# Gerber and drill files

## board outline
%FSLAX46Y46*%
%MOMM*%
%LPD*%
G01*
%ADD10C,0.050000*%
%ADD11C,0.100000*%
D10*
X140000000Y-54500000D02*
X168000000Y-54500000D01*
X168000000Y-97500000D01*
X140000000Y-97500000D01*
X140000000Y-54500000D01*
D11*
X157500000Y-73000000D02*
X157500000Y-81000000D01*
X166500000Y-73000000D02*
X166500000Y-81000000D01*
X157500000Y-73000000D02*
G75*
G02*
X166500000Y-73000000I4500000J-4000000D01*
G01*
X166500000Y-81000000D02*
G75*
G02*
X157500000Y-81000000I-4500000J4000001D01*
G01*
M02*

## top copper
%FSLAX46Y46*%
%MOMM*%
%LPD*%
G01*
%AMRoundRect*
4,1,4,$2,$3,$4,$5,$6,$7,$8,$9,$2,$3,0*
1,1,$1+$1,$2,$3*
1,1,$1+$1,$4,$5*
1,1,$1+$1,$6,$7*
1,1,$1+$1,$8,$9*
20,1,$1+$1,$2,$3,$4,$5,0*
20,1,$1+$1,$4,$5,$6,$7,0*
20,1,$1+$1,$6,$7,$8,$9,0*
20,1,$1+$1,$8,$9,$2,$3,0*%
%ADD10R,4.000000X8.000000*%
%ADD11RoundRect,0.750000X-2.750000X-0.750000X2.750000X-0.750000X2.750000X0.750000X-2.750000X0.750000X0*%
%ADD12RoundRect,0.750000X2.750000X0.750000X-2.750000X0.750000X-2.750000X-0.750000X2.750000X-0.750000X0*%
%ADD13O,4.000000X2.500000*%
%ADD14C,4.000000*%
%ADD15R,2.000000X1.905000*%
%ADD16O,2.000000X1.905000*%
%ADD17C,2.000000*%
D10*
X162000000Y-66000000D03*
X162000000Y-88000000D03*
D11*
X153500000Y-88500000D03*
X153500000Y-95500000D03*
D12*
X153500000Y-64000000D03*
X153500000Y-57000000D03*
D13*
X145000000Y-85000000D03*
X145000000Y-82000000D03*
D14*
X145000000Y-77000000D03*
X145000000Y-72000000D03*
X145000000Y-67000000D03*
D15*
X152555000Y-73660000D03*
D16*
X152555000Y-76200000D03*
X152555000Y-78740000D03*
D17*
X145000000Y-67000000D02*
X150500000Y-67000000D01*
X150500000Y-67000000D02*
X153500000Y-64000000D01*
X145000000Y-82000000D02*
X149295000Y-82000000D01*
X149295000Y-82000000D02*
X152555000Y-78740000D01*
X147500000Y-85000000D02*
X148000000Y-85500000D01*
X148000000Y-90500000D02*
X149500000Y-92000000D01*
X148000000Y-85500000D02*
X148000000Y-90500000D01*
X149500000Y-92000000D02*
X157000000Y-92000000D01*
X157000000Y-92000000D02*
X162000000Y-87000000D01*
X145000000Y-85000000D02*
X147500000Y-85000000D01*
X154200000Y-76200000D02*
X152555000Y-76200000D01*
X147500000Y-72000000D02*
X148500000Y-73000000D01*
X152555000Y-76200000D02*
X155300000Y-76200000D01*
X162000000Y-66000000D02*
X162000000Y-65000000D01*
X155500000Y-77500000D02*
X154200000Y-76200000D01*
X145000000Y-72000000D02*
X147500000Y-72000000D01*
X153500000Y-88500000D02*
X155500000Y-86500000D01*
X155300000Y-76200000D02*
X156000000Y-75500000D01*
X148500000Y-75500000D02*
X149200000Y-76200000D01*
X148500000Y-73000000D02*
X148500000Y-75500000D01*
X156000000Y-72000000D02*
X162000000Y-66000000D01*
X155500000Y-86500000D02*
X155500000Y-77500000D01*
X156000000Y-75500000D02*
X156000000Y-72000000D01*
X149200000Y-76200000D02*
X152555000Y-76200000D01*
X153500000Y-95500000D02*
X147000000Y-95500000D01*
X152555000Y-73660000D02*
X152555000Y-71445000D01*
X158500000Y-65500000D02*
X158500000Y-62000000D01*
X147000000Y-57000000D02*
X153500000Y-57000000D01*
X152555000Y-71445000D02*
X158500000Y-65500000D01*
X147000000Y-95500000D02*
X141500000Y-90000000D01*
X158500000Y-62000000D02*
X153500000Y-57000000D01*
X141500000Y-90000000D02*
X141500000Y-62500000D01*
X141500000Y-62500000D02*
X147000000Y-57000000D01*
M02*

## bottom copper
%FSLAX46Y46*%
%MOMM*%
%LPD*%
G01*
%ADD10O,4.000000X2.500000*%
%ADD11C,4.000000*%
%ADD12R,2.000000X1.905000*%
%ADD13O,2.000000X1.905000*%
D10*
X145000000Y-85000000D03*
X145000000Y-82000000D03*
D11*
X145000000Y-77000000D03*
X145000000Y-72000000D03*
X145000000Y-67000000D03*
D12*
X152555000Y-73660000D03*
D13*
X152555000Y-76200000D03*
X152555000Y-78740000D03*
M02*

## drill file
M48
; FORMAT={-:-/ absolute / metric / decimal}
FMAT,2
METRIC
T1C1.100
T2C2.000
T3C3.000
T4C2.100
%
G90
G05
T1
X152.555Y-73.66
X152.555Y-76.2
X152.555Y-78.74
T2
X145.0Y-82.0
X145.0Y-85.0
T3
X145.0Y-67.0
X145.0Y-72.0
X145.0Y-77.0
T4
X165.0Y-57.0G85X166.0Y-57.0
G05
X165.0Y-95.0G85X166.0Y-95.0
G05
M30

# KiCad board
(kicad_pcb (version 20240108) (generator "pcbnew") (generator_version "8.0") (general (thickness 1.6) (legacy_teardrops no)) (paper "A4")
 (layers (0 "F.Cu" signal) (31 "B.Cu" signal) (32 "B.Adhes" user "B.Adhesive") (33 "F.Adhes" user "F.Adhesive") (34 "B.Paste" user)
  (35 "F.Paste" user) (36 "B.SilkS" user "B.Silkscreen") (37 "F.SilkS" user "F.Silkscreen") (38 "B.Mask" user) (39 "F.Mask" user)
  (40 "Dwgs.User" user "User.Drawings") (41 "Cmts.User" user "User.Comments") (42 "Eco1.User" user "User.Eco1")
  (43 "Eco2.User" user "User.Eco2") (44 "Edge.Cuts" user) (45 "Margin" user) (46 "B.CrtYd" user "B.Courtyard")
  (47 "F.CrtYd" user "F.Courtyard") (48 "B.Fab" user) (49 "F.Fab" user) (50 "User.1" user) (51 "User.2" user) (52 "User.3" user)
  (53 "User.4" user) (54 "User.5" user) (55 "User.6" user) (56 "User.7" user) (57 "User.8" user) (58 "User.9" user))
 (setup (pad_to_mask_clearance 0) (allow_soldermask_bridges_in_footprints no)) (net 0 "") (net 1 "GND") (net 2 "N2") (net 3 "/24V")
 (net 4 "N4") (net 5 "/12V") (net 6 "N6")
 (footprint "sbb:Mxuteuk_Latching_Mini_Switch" (layer "F.Cu") (at 162 77 -90)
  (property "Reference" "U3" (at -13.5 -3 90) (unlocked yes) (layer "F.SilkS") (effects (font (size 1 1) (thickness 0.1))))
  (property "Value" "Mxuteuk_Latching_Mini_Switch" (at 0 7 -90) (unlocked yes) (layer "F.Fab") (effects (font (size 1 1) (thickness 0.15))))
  (fp_line (start -4 4.5) (end 4 4.5) (stroke (width 0.1) (type default)) (layer "Edge.Cuts"))
  (fp_line (start -4 -4.5) (end 4 -4.5) (stroke (width 0.1) (type default)) (layer "Edge.Cuts"))
  (fp_arc (start -4 4.5) (mid -6.020797 0) (end -4 -4.5) (stroke (width 0.1) (type default)) (layer "Edge.Cuts"))
  (fp_arc (start 4 -4.5) (mid 6.020797 0) (end 4 4.5) (stroke (width 0.1) (type default)) (layer "Edge.Cuts"))
  (pad "1" smd rect (at -11 0 270) (size 8 4) (layers "F.Cu" "F.Paste" "F.Mask") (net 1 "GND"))
  (pad "2" smd rect (at 11 0 270) (size 8 4) (layers "F.Cu" "F.Paste" "F.Mask") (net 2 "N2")))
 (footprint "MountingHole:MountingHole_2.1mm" (layer "F.Cu") (at 165.5 57)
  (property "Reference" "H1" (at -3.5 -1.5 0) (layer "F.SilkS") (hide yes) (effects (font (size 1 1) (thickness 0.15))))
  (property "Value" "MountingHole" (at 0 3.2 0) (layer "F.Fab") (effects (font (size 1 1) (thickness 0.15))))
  (pad "" np_thru_hole oval (at 0 0) (size 3.1 2.1) (drill oval 3.1 2.1) (layers "F&B.Cu" "*.Mask")))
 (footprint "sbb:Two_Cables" (layer "F.Cu") (at 153.5 92.5)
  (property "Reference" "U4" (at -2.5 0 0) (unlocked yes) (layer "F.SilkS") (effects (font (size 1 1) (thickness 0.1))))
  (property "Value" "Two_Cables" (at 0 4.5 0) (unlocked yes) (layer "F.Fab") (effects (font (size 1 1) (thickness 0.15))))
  (pad "1" smd roundrect (at 0 -4) (size 7 3) (layers "F.Cu" "F.Paste" "F.Mask") (roundrect_rratio 0.25) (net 1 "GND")
   (thermal_bridge_angle 45))
  (pad "2" smd roundrect (at 0 3) (size 7 3) (layers "F.Cu" "F.Paste" "F.Mask") (roundrect_rratio 0.25) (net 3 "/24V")
   (thermal_bridge_angle 45)))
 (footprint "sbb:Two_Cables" (layer "F.Cu") (at 153.5 60 180)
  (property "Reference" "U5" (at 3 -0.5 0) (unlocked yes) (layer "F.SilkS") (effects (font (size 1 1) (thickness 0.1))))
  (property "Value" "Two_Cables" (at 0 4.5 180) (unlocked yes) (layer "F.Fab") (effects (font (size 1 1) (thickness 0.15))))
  (pad "1" smd roundrect (at 0 -4 180) (size 7 3) (layers "F.Cu" "F.Paste" "F.Mask") (roundrect_rratio 0.25) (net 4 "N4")
   (thermal_bridge_angle 45))
  (pad "2" smd roundrect (at 0 3 180) (size 7 3) (layers "F.Cu" "F.Paste" "F.Mask") (roundrect_rratio 0.25) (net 3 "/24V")
   (thermal_bridge_angle 45)))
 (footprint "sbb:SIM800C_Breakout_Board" (layer "F.Cu") (at 145 85)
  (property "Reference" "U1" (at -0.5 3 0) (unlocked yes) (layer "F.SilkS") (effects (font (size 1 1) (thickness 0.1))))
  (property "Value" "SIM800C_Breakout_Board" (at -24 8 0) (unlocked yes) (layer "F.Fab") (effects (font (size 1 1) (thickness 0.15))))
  (pad "1" thru_hole oval (at 0 0) (size 4 2.5) (drill 2) (layers "*.Cu" "*.Mask") (remove_unused_layers no) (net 2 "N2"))
  (pad "2" thru_hole oval (at 0 -3) (size 4 2.5) (drill 2) (layers "*.Cu" "*.Mask") (remove_unused_layers no) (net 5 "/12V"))
  (pad "3" thru_hole circle (at 0 -8) (size 4 4) (drill 3) (layers "*.Cu" "*.Mask") (remove_unused_layers no) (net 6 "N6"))
  (pad "4" thru_hole circle (at 0 -13) (size 4 4) (drill 3) (layers "*.Cu" "*.Mask") (remove_unused_layers no) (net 1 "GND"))
  (pad "5" thru_hole circle (at 0 -18) (size 4 4) (drill 3) (layers "*.Cu" "*.Mask") (remove_unused_layers no) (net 4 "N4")))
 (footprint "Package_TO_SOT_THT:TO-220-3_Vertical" (layer "F.Cu") (at 152.555 73.66 -90)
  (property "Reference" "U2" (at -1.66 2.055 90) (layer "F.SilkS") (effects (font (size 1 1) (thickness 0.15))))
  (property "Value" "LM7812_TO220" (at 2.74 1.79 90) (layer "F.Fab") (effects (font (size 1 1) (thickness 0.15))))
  (pad "1" thru_hole rect (at 0 0 270) (size 1.905 2) (drill 1.1) (layers "*.Cu" "*.Mask") (remove_unused_layers no) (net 3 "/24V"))
  (pad "2" thru_hole oval (at 2.54 0 270) (size 1.905 2) (drill 1.1) (layers "*.Cu" "*.Mask") (remove_unused_layers no) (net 1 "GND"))
  (pad "3" thru_hole oval (at 5.08 0 270) (size 1.905 2) (drill 1.1) (layers "*.Cu" "*.Mask") (remove_unused_layers no) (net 5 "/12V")))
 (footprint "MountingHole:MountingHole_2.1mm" (layer "F.Cu") (at 165.5 95)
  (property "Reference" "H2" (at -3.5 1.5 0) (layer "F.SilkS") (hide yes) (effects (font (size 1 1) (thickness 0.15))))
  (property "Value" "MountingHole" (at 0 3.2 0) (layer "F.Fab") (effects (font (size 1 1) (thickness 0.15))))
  (pad "" np_thru_hole oval (at 0 0) (size 3.1 2.1) (drill oval 3.1 2.1) (layers "F&B.Cu" "*.Mask")))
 (gr_rect (start 140 54.5) (end 168 97.5) (stroke (width 0.05) (type default)) (fill none) (layer "Edge.Cuts"))
 (segment (start 145 67) (end 150.5 67) (width 2) (layer "F.Cu") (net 4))
 (segment (start 150.5 67) (end 153.5 64) (width 2) (layer "F.Cu") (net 4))
 (segment (start 145 82) (end 149.295 82) (width 2) (layer "F.Cu") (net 5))
 (segment (start 149.295 82) (end 152.555 78.74) (width 2) (layer "F.Cu") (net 5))
 (segment (start 147.5 85) (end 148 85.5) (width 2) (layer "F.Cu") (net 2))
 (segment (start 148 90.5) (end 149.5 92) (width 2) (layer "F.Cu") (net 2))
 (segment (start 148 85.5) (end 148 90.5) (width 2) (layer "F.Cu") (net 2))
 (segment (start 149.5 92) (end 157 92) (width 2) (layer "F.Cu") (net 2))
 (segment (start 157 92) (end 162 87) (width 2) (layer "F.Cu") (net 2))
 (segment (start 145 85) (end 147.5 85) (width 2) (layer "F.Cu") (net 2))
 (segment (start 154.2 76.2) (end 152.555 76.2) (width 2) (layer "F.Cu") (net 1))
 (segment (start 147.5 72) (end 148.5 73) (width 2) (layer "F.Cu") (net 1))
 (segment (start 152.555 76.2) (end 155.3 76.2) (width 2) (layer "F.Cu") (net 1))
 (segment (start 162 66) (end 162 65) (width 2) (layer "F.Cu") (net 1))
 (segment (start 155.5 77.5) (end 154.2 76.2) (width 2) (layer "F.Cu") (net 1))
 (segment (start 145 72) (end 147.5 72) (width 2) (layer "F.Cu") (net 1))
 (segment (start 153.5 88.5) (end 155.5 86.5) (width 2) (layer "F.Cu") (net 1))
 (segment (start 155.3 76.2) (end 156 75.5) (width 2) (layer "F.Cu") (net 1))
 (segment (start 148.5 75.5) (end 149.2 76.2) (width 2) (layer "F.Cu") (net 1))
 (segment (start 148.5 73) (end 148.5 75.5) (width 2) (layer "F.Cu") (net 1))
 (segment (start 156 72) (end 162 66) (width 2) (layer "F.Cu") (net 1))
 (segment (start 155.5 86.5) (end 155.5 77.5) (width 2) (layer "F.Cu") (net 1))
 (segment (start 156 75.5) (end 156 72) (width 2) (layer "F.Cu") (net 1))
 (segment (start 149.2 76.2) (end 152.555 76.2) (width 2) (layer "F.Cu") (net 1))
 (segment (start 153.5 95.5) (end 147 95.5) (width 2) (layer "F.Cu") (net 3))
 (segment (start 152.555 73.66) (end 152.555 71.445) (width 2) (layer "F.Cu") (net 3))
 (segment (start 158.5 65.5) (end 158.5 62) (width 2) (layer "F.Cu") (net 3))
 (segment (start 147 57) (end 153.5 57) (width 2) (layer "F.Cu") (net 3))
 (segment (start 152.555 71.445) (end 158.5 65.5) (width 2) (layer "F.Cu") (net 3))
 (segment (start 147 95.5) (end 141.5 90) (width 2) (layer "F.Cu") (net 3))
 (segment (start 158.5 62) (end 153.5 57) (width 2) (layer "F.Cu") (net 3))
 (segment (start 141.5 90) (end 141.5 62.5) (width 2) (layer "F.Cu") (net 3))
 (segment (start 141.5 62.5) (end 147 57) (width 2) (layer "F.Cu") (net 3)))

